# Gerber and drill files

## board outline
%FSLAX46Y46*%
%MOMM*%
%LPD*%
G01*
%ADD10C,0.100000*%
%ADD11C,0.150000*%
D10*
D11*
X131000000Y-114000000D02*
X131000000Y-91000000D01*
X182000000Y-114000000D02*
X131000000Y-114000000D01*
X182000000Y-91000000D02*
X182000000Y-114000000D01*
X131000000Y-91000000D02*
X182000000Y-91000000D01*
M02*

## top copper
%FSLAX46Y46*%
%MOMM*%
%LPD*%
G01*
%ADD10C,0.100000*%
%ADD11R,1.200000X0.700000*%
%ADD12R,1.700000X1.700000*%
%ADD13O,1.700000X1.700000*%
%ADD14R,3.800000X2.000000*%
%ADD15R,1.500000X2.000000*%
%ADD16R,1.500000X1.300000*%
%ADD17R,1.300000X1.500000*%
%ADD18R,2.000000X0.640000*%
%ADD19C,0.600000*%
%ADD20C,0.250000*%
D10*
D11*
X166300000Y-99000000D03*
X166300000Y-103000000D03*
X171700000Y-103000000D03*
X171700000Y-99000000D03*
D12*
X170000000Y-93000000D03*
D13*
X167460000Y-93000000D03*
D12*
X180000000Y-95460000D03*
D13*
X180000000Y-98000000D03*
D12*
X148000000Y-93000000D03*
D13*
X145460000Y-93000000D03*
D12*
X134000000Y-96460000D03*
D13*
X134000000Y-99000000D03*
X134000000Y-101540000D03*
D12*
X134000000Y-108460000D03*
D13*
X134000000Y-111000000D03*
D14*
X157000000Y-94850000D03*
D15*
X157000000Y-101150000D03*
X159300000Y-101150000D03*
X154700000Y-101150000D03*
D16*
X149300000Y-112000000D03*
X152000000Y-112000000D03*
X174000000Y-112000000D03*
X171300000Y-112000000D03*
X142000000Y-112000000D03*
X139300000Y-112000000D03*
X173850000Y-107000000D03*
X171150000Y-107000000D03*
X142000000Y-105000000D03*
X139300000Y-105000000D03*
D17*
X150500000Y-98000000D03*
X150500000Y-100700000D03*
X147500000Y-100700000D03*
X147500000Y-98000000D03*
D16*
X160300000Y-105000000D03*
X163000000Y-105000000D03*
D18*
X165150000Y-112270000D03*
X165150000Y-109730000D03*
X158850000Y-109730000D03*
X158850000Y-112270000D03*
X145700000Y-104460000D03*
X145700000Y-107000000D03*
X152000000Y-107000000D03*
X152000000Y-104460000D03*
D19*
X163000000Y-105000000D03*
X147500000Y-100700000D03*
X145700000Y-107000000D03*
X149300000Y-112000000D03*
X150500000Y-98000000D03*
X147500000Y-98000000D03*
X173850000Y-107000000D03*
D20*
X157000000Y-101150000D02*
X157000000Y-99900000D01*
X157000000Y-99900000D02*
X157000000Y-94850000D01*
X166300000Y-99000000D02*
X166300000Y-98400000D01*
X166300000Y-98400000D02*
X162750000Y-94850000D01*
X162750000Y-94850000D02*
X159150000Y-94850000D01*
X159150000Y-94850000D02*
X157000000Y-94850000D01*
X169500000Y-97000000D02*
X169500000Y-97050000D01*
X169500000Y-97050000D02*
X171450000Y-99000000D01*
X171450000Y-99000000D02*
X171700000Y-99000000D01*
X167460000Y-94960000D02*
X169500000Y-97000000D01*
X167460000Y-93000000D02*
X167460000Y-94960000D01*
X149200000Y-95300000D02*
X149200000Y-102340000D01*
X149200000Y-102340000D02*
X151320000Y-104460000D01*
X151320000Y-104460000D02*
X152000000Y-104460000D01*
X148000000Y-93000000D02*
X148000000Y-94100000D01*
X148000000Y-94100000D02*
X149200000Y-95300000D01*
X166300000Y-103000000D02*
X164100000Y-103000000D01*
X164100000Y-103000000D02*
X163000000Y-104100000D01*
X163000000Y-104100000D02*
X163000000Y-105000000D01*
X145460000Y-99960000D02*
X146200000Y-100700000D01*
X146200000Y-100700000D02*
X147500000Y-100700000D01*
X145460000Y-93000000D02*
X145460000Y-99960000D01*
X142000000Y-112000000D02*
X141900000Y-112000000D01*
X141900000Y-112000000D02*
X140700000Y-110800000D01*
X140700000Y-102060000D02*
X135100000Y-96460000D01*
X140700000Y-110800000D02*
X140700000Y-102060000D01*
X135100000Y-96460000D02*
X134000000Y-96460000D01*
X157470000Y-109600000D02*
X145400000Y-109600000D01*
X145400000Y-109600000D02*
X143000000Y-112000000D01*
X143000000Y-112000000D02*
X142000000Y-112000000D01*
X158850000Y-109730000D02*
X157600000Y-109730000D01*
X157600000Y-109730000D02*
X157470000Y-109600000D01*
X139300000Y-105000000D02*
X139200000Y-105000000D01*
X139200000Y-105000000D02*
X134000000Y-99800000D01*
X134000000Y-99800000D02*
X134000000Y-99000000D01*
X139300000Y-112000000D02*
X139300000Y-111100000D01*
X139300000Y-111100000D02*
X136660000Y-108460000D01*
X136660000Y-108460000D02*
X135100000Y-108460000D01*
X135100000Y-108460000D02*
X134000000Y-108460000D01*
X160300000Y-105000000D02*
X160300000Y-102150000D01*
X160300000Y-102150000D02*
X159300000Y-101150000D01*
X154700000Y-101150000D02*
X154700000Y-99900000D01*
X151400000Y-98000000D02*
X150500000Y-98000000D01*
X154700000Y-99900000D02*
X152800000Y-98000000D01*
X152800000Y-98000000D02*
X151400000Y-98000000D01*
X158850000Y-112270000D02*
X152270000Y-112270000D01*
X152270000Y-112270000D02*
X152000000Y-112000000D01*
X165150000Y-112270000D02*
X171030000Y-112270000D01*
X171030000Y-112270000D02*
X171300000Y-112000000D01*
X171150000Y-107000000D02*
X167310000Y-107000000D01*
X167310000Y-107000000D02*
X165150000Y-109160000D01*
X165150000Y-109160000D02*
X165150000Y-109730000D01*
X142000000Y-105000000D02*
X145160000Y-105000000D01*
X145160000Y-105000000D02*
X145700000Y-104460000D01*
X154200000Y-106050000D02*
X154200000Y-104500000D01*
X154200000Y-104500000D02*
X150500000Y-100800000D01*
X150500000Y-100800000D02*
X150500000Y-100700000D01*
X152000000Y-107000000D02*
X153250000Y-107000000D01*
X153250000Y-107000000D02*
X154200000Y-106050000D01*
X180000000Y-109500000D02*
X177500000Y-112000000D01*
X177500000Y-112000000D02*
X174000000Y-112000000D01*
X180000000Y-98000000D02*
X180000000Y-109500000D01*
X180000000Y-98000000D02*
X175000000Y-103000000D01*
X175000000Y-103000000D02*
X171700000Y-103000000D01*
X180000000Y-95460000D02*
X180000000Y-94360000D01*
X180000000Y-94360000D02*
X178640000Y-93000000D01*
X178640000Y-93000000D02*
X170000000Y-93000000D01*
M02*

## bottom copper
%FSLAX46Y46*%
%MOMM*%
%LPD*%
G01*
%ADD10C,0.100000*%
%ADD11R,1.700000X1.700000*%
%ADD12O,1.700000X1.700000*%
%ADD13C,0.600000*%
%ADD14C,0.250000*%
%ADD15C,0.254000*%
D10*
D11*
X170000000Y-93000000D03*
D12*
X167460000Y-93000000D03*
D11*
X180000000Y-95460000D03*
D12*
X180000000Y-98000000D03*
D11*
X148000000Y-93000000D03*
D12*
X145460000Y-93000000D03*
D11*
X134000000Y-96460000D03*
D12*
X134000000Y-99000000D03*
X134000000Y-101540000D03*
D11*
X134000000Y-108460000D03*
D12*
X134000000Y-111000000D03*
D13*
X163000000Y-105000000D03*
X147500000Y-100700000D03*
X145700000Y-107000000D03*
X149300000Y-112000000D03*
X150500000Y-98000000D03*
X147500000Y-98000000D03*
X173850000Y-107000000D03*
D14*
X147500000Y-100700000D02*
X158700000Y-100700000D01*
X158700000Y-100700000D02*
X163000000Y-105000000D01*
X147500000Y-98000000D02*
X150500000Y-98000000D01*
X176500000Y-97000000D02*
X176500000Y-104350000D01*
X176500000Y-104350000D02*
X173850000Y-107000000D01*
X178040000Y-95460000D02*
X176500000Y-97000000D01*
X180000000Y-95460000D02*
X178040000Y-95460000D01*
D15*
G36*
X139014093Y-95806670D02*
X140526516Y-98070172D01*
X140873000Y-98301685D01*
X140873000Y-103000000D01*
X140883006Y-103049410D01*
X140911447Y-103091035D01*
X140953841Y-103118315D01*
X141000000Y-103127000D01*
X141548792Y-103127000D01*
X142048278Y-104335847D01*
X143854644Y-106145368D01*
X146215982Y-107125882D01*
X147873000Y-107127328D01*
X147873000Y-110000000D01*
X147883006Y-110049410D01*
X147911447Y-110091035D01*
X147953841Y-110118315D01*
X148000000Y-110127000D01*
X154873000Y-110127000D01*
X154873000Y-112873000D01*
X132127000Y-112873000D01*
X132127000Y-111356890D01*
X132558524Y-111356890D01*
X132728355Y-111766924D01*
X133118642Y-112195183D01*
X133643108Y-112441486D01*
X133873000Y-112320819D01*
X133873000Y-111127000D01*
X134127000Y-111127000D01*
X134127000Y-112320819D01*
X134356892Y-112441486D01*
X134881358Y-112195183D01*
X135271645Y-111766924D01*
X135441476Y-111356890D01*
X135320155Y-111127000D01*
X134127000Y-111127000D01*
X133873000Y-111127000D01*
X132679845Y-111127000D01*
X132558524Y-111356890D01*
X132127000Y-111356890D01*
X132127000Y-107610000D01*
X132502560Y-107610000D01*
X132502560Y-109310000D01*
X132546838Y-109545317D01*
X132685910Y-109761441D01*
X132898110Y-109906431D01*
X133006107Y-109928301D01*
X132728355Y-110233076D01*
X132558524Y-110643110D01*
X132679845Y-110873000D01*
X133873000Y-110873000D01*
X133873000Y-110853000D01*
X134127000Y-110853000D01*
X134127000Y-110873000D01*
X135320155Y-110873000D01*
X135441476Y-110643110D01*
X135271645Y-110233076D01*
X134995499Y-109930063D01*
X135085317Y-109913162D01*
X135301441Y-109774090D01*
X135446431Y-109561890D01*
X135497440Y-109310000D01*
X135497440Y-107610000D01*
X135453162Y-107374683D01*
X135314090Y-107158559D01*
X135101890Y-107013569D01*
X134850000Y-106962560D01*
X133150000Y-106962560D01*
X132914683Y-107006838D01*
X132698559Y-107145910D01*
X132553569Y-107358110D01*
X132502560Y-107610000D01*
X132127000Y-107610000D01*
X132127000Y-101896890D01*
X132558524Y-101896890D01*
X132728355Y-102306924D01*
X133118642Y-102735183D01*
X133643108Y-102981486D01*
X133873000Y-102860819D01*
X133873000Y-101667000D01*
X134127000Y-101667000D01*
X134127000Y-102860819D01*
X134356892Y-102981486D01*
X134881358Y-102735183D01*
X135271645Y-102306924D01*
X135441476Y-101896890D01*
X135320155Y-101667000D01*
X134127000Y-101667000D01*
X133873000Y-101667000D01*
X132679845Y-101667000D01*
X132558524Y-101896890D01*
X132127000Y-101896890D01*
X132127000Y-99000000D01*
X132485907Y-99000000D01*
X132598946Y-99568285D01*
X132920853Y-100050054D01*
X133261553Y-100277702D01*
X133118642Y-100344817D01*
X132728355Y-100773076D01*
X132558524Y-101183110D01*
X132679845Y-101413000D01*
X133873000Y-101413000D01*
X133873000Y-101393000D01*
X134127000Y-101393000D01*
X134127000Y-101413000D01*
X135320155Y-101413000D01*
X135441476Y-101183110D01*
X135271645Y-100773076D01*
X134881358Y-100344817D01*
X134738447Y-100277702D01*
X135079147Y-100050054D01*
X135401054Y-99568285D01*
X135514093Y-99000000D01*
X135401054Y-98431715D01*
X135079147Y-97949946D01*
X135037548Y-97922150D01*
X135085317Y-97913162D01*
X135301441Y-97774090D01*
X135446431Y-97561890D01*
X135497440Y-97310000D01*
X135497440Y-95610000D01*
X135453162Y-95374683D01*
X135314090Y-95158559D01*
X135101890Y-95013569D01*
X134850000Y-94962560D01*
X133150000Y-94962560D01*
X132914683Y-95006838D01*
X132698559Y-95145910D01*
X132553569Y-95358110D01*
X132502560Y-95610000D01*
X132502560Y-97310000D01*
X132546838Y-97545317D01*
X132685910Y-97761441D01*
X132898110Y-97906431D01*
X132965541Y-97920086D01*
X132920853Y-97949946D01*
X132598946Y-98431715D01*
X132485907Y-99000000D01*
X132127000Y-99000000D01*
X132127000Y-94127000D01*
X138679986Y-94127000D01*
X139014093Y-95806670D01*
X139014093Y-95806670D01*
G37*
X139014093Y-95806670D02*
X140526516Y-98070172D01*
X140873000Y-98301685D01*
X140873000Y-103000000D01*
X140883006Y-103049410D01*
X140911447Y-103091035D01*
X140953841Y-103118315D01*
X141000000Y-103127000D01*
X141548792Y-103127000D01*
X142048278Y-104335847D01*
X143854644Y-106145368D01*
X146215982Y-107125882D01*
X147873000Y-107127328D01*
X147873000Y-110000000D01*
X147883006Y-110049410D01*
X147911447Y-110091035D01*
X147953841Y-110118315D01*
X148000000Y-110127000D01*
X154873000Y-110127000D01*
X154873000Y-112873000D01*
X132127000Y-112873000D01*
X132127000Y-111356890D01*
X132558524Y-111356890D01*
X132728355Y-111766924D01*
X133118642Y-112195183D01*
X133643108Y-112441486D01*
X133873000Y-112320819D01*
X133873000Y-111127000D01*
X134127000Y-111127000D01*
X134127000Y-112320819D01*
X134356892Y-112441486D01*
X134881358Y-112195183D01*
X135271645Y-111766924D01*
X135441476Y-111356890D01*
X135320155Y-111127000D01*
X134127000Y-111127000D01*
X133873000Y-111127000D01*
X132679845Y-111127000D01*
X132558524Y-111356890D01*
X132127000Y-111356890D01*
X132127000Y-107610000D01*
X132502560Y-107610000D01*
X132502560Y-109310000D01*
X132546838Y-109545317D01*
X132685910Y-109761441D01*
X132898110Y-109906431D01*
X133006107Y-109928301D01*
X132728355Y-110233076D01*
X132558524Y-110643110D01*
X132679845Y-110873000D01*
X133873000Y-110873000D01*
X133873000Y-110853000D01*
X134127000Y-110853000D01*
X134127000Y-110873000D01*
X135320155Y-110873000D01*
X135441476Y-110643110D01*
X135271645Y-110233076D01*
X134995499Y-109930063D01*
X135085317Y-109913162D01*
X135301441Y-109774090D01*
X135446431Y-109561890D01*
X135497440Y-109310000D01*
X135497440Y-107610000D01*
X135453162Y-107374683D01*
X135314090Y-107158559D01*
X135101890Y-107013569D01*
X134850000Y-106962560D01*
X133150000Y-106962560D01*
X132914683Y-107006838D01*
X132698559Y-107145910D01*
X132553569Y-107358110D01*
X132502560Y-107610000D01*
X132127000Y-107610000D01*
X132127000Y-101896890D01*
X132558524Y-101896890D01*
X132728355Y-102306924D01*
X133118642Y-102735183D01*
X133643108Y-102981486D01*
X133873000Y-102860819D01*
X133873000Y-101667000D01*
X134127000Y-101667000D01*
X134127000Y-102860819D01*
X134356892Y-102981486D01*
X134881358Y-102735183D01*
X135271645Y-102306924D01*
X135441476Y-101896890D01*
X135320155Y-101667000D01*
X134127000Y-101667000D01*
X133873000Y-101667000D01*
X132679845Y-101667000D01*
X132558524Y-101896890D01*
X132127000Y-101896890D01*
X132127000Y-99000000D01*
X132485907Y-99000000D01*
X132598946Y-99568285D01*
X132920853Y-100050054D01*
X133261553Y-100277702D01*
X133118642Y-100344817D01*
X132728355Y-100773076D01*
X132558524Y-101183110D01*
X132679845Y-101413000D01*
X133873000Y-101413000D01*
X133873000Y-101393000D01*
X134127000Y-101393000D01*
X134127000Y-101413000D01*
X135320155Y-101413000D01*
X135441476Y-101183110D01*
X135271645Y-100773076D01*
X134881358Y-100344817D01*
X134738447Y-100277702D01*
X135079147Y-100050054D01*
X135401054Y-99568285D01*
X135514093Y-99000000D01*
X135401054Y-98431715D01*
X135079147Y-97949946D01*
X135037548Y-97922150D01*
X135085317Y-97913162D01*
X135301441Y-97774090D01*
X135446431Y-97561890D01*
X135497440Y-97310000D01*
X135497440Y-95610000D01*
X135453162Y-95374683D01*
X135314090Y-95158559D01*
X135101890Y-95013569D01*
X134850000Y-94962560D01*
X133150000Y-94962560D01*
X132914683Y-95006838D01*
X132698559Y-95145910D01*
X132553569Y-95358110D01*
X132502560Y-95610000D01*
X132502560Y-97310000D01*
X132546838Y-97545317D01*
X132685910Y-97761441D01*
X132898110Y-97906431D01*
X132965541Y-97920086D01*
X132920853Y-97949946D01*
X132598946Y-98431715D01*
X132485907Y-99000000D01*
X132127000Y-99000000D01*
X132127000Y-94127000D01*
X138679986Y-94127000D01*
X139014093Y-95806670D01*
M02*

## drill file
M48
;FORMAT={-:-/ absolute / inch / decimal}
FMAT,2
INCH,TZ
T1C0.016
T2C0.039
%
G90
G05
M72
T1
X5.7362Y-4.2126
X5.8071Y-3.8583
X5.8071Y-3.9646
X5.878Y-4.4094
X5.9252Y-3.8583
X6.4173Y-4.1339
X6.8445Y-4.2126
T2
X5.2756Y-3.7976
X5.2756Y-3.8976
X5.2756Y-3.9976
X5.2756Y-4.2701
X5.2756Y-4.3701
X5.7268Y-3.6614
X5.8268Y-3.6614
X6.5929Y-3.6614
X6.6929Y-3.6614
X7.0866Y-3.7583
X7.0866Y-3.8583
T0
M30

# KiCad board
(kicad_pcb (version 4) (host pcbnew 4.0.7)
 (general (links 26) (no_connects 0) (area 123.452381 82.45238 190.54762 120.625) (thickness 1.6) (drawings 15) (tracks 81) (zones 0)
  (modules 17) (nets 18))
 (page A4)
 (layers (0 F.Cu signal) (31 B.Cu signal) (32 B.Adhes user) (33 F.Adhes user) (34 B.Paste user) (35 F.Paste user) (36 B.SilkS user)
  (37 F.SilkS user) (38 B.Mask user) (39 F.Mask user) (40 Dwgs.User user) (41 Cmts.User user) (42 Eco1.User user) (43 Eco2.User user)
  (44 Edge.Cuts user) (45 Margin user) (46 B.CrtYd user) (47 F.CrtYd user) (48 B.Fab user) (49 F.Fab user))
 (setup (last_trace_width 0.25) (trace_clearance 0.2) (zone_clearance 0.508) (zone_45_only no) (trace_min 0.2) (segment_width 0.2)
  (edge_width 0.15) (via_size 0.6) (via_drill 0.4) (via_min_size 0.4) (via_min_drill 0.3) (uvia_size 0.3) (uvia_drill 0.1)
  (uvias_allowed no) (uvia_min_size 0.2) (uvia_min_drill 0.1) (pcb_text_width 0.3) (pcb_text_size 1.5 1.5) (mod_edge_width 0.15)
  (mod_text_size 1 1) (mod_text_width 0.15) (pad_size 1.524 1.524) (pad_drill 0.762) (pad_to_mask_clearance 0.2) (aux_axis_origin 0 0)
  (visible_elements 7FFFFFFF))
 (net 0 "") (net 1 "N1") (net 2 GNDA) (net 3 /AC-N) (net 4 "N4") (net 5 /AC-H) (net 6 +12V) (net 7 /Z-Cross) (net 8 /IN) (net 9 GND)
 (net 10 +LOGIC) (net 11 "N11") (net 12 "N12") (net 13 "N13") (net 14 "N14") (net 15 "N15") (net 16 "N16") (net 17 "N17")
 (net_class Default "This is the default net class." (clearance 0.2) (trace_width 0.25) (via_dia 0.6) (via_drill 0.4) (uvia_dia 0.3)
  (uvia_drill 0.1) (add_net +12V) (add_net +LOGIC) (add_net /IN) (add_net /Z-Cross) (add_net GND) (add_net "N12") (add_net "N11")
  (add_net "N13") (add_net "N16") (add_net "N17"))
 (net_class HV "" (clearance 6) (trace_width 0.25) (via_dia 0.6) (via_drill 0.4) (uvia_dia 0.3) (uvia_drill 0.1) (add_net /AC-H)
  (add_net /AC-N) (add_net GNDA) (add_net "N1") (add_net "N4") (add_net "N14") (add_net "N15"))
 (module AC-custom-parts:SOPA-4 (layer F.Cu) (at 169 101)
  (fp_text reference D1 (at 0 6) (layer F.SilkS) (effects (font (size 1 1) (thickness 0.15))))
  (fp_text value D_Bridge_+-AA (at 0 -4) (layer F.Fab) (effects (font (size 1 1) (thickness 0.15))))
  (pad 1 smd rect (at -2.7 -2) (size 1.2 0.7) (layers F.Cu F.Paste F.Mask) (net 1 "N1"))
  (pad 2 smd rect (at -2.7 2) (size 1.2 0.7) (layers F.Cu F.Paste F.Mask) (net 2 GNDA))
  (pad 3 smd rect (at 2.7 2) (size 1.2 0.7) (layers F.Cu F.Paste F.Mask) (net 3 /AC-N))
  (pad 4 smd rect (at 2.7 -2) (size 1.2 0.7) (layers F.Cu F.Paste F.Mask) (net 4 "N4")))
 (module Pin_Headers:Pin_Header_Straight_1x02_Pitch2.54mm (layer F.Cu) (at 170 93 270)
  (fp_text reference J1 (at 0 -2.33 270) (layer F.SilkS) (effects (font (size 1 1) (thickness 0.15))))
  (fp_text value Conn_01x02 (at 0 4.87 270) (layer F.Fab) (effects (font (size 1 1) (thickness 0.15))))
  (pad 1 thru_hole rect (at 0 0 270) (size 1.7 1.7) (drill 1) (layers *.Cu *.Mask) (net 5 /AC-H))
  (pad 2 thru_hole oval (at 0 2.54 270) (size 1.7 1.7) (drill 1) (layers *.Cu *.Mask) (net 4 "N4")))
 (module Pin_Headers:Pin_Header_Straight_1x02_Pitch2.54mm (layer F.Cu) (at 180 95.46)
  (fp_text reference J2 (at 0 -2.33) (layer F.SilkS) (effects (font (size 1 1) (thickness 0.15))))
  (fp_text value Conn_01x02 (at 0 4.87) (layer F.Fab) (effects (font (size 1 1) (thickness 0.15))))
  (pad 1 thru_hole rect (at 0 0) (size 1.7 1.7) (drill 1) (layers *.Cu *.Mask) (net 5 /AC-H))
  (pad 2 thru_hole oval (at 0 2.54) (size 1.7 1.7) (drill 1) (layers *.Cu *.Mask) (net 3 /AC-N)))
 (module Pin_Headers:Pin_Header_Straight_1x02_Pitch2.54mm (layer F.Cu) (at 148 93 270)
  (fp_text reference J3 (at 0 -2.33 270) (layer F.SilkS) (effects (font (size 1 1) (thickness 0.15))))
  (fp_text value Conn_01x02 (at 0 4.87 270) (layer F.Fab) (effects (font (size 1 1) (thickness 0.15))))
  (pad 1 thru_hole rect (at 0 0 270) (size 1.7 1.7) (drill 1) (layers *.Cu *.Mask) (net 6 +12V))
  (pad 2 thru_hole oval (at 0 2.54 270) (size 1.7 1.7) (drill 1) (layers *.Cu *.Mask) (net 2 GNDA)))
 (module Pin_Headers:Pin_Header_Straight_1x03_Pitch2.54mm (layer F.Cu) (at 134 96.46)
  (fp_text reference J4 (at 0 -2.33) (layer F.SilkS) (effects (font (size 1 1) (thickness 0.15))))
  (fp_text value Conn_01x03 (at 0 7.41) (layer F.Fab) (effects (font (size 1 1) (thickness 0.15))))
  (pad 1 thru_hole rect (at 0 0) (size 1.7 1.7) (drill 1) (layers *.Cu *.Mask) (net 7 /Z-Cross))
  (pad 2 thru_hole oval (at 0 2.54) (size 1.7 1.7) (drill 1) (layers *.Cu *.Mask) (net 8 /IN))
  (pad 3 thru_hole oval (at 0 5.08) (size 1.7 1.7) (drill 1) (layers *.Cu *.Mask) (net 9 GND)))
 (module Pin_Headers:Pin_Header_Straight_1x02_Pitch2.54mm (layer F.Cu) (at 134 108.46)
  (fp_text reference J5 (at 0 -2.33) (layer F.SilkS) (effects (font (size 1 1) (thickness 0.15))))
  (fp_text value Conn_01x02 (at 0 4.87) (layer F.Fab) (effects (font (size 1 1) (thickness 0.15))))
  (pad 1 thru_hole rect (at 0 0) (size 1.7 1.7) (drill 1) (layers *.Cu *.Mask) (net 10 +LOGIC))
  (pad 2 thru_hole oval (at 0 2.54) (size 1.7 1.7) (drill 1) (layers *.Cu *.Mask) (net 9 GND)))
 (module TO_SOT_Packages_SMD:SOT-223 (layer F.Cu) (at 157 98 90)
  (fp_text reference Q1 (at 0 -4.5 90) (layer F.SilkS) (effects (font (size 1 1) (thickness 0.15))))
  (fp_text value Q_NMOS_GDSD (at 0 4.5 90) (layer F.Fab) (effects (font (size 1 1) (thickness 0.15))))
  (pad 4 smd rect (at 3.15 0 90) (size 2 3.8) (layers F.Cu F.Paste F.Mask) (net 1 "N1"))
  (pad 2 smd rect (at -3.15 0 90) (size 2 1.5) (layers F.Cu F.Paste F.Mask) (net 1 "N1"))
  (pad 3 smd rect (at -3.15 2.3 90) (size 2 1.5) (layers F.Cu F.Paste F.Mask) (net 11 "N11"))
  (pad 1 smd rect (at -3.15 -2.3 90) (size 2 1.5) (layers F.Cu F.Paste F.Mask) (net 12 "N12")))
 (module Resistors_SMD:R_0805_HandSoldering (layer F.Cu) (at 150.65 112)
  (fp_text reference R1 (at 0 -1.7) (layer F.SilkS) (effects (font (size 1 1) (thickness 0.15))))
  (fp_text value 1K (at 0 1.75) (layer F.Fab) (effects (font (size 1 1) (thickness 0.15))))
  (pad 1 smd rect (at -1.35 0) (size 1.5 1.3) (layers F.Cu F.Paste F.Mask) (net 9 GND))
  (pad 2 smd rect (at 1.35 0) (size 1.5 1.3) (layers F.Cu F.Paste F.Mask) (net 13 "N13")))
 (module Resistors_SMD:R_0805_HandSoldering (layer F.Cu) (at 172.65 112 180)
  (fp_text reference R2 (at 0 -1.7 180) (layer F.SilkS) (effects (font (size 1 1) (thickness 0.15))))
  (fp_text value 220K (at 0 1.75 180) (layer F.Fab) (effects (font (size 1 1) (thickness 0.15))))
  (pad 1 smd rect (at -1.35 0 180) (size 1.5 1.3) (layers F.Cu F.Paste F.Mask) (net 3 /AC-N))
  (pad 2 smd rect (at 1.35 0 180) (size 1.5 1.3) (layers F.Cu F.Paste F.Mask) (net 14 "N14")))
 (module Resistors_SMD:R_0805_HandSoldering (layer F.Cu) (at 140.65 112 180)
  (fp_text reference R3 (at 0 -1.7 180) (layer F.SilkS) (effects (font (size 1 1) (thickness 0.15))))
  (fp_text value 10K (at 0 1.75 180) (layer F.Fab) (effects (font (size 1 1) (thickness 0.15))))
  (pad 1 smd rect (at -1.35 0 180) (size 1.5 1.3) (layers F.Cu F.Paste F.Mask) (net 7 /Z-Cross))
  (pad 2 smd rect (at 1.35 0 180) (size 1.5 1.3) (layers F.Cu F.Paste F.Mask) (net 10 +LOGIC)))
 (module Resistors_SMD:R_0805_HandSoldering (layer F.Cu) (at 172.5 107 180)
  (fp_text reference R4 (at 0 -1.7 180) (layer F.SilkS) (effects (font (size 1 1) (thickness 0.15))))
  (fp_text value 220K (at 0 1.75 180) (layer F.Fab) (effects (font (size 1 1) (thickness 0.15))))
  (pad 1 smd rect (at -1.35 0 180) (size 1.5 1.3) (layers F.Cu F.Paste F.Mask) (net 5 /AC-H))
  (pad 2 smd rect (at 1.35 0 180) (size 1.5 1.3) (layers F.Cu F.Paste F.Mask) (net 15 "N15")))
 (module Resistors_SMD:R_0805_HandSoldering (layer F.Cu) (at 140.65 105 180)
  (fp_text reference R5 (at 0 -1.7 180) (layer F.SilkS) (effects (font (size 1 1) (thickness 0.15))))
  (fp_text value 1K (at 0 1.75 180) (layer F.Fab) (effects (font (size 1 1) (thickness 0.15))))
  (pad 1 smd rect (at -1.35 0 180) (size 1.5 1.3) (layers F.Cu F.Paste F.Mask) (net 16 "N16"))
  (pad 2 smd rect (at 1.35 0 180) (size 1.5 1.3) (layers F.Cu F.Paste F.Mask) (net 8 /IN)))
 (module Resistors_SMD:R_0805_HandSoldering (layer F.Cu) (at 150.5 99.35 270)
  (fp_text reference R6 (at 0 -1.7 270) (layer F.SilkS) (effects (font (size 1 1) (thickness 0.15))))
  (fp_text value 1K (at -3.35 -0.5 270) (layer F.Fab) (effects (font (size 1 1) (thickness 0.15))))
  (pad 1 smd rect (at -1.35 0 270) (size 1.5 1.3) (layers F.Cu F.Paste F.Mask) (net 12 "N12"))
  (pad 2 smd rect (at 1.35 0 270) (size 1.5 1.3) (layers F.Cu F.Paste F.Mask) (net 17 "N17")))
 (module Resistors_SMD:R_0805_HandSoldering (layer F.Cu) (at 147.5 99.35 90)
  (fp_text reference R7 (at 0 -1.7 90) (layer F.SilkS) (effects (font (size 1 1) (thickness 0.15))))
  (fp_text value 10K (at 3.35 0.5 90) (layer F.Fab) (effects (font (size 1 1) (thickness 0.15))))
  (pad 1 smd rect (at -1.35 0 90) (size 1.5 1.3) (layers F.Cu F.Paste F.Mask) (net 2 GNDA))
  (pad 2 smd rect (at 1.35 0 90) (size 1.5 1.3) (layers F.Cu F.Paste F.Mask) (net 12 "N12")))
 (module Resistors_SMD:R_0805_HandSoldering (layer F.Cu) (at 161.65 105)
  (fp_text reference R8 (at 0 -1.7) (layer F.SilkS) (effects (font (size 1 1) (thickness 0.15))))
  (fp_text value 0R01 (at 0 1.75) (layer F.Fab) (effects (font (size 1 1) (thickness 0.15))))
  (pad 1 smd rect (at -1.35 0) (size 1.5 1.3) (layers F.Cu F.Paste F.Mask) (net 11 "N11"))
  (pad 2 smd rect (at 1.35 0) (size 1.5 1.3) (layers F.Cu F.Paste F.Mask) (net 2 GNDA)))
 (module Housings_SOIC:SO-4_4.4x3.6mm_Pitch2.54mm (layer F.Cu) (at 162 111 180)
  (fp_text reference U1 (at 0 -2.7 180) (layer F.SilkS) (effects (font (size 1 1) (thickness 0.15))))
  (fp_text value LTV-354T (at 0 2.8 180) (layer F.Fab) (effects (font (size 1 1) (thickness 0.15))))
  (pad 1 smd rect (at -3.15 -1.27 180) (size 2 0.64) (layers F.Cu F.Paste F.Mask) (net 14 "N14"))
  (pad 2 smd rect (at -3.15 1.27 180) (size 2 0.64) (layers F.Cu F.Paste F.Mask) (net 15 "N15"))
  (pad 3 smd rect (at 3.15 1.27 180) (size 2 0.64) (layers F.Cu F.Paste F.Mask) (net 7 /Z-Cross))
  (pad 4 smd rect (at 3.15 -1.27 180) (size 2 0.64) (layers F.Cu F.Paste F.Mask) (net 13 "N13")))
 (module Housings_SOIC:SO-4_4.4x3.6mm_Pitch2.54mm (layer F.Cu) (at 148.85 105.73)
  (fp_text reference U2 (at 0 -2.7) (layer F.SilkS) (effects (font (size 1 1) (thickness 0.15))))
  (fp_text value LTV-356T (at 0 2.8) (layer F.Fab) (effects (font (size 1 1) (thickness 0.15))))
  (pad 1 smd rect (at -3.15 -1.27) (size 2 0.64) (layers F.Cu F.Paste F.Mask) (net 16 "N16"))
  (pad 2 smd rect (at -3.15 1.27) (size 2 0.64) (layers F.Cu F.Paste F.Mask) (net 9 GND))
  (pad 3 smd rect (at 3.15 1.27) (size 2 0.64) (layers F.Cu F.Paste F.Mask) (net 17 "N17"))
  (pad 4 smd rect (at 3.15 -1.27) (size 2 0.64) (layers F.Cu F.Paste F.Mask) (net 6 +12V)))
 (gr_line (start 131 114) (end 131 91) (layer Edge.Cuts) (width 0.15))
 (gr_line (start 182 114) (end 131 114) (layer Edge.Cuts) (width 0.15))
 (gr_line (start 182 91) (end 182 114) (layer Edge.Cuts) (width 0.15))
 (gr_line (start 131 91) (end 182 91) (layer Edge.Cuts) (width 0.15))
 (segment (start 157 101.15) (end 157 99.9) (width 0.25) (layer F.Cu) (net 1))
 (segment (start 157 99.9) (end 157 94.85) (width 0.25) (layer F.Cu) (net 1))
 (segment (start 166.3 99) (end 166.3 98.4) (width 0.25) (layer F.Cu) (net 1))
 (segment (start 166.3 98.4) (end 162.75 94.85) (width 0.25) (layer F.Cu) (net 1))
 (segment (start 162.75 94.85) (end 159.15 94.85) (width 0.25) (layer F.Cu) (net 1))
 (segment (start 159.15 94.85) (end 157 94.85) (width 0.25) (layer F.Cu) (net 1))
 (segment (start 169.5 97) (end 169.5 97.05) (width 0.25) (layer F.Cu) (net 4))
 (segment (start 169.5 97.05) (end 171.45 99) (width 0.25) (layer F.Cu) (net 4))
 (segment (start 171.45 99) (end 171.7 99) (width 0.25) (layer F.Cu) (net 4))
 (segment (start 167.46 94.96) (end 169.5 97) (width 0.25) (layer F.Cu) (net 4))
 (segment (start 167.46 93) (end 167.46 94.96) (width 0.25) (layer F.Cu) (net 4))
 (segment (start 149.2 95.3) (end 149.2 102.34) (width 0.25) (layer F.Cu) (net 6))
 (segment (start 149.2 102.34) (end 151.32 104.46) (width 0.25) (layer F.Cu) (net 6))
 (segment (start 151.32 104.46) (end 152 104.46) (width 0.25) (layer F.Cu) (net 6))
 (segment (start 148 93) (end 148 94.1) (width 0.25) (layer F.Cu) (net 6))
 (segment (start 148 94.1) (end 149.2 95.3) (width 0.25) (layer F.Cu) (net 6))
 (segment (start 147.5 100.7) (end 158.7 100.7) (width 0.25) (layer B.Cu) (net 2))
 (via (at 163 105) (size 0.6) (drill 0.4) (layers F.Cu B.Cu) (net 2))
 (segment (start 158.7 100.7) (end 163 105) (width 0.25) (layer B.Cu) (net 2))
 (via (at 147.5 100.7) (size 0.6) (drill 0.4) (layers F.Cu B.Cu) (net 2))
 (segment (start 166.3 103) (end 164.1 103) (width 0.25) (layer F.Cu) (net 2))
 (segment (start 164.1 103) (end 163 104.1) (width 0.25) (layer F.Cu) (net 2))
 (segment (start 163 104.1) (end 163 105) (width 0.25) (layer F.Cu) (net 2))
 (segment (start 145.46 99.96) (end 146.2 100.7) (width 0.25) (layer F.Cu) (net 2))
 (segment (start 146.2 100.7) (end 147.5 100.7) (width 0.25) (layer F.Cu) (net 2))
 (segment (start 145.46 93) (end 145.46 99.96) (width 0.25) (layer F.Cu) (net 2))
 (segment (start 142 112) (end 141.9 112) (width 0.25) (layer F.Cu) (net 7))
 (segment (start 141.9 112) (end 140.7 110.8) (width 0.25) (layer F.Cu) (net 7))
 (segment (start 140.7 102.06) (end 135.1 96.46) (width 0.25) (layer F.Cu) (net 7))
 (segment (start 140.7 110.8) (end 140.7 102.06) (width 0.25) (layer F.Cu) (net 7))
 (segment (start 135.1 96.46) (end 134 96.46) (width 0.25) (layer F.Cu) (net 7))
 (segment (start 157.47 109.6) (end 145.4 109.6) (width 0.25) (layer F.Cu) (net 7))
 (segment (start 145.4 109.6) (end 143 112) (width 0.25) (layer F.Cu) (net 7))
 (segment (start 143 112) (end 142 112) (width 0.25) (layer F.Cu) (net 7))
 (segment (start 158.85 109.73) (end 157.6 109.73) (width 0.25) (layer F.Cu) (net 7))
 (segment (start 157.6 109.73) (end 157.47 109.6) (width 0.25) (layer F.Cu) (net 7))
 (segment (start 139.3 105) (end 139.2 105) (width 0.25) (layer F.Cu) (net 8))
 (segment (start 139.2 105) (end 134 99.8) (width 0.25) (layer F.Cu) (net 8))
 (segment (start 134 99.8) (end 134 99) (width 0.25) (layer F.Cu) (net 8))
 (via (at 145.7 107) (size 0.6) (drill 0.4) (layers F.Cu B.Cu) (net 9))
 (via (at 149.3 112) (size 0.6) (drill 0.4) (layers F.Cu B.Cu) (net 9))
 (segment (start 139.3 112) (end 139.3 111.1) (width 0.25) (layer F.Cu) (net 10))
 (segment (start 139.3 111.1) (end 136.66 108.46) (width 0.25) (layer F.Cu) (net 10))
 (segment (start 136.66 108.46) (end 135.1 108.46) (width 0.25) (layer F.Cu) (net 10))
 (segment (start 135.1 108.46) (end 134 108.46) (width 0.25) (layer F.Cu) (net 10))
 (segment (start 160.3 105) (end 160.3 102.15) (width 0.25) (layer F.Cu) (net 11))
 (segment (start 160.3 102.15) (end 159.3 101.15) (width 0.25) (layer F.Cu) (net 11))
 (segment (start 147.5 98) (end 150.5 98) (width 0.25) (layer B.Cu) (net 12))
 (via (at 150.5 98) (size 0.6) (drill 0.4) (layers F.Cu B.Cu) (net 12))
 (via (at 147.5 98) (size 0.6) (drill 0.4) (layers F.Cu B.Cu) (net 12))
 (segment (start 154.7 101.15) (end 154.7 99.9) (width 0.25) (layer F.Cu) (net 12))
 (segment (start 151.4 98) (end 150.5 98) (width 0.25) (layer F.Cu) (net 12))
 (segment (start 154.7 99.9) (end 152.8 98) (width 0.25) (layer F.Cu) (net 12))
 (segment (start 152.8 98) (end 151.4 98) (width 0.25) (layer F.Cu) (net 12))
 (segment (start 158.85 112.27) (end 152.27 112.27) (width 0.25) (layer F.Cu) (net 13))
 (segment (start 152.27 112.27) (end 152 112) (width 0.25) (layer F.Cu) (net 13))
 (segment (start 165.15 112.27) (end 171.03 112.27) (width 0.25) (layer F.Cu) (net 14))
 (segment (start 171.03 112.27) (end 171.3 112) (width 0.25) (layer F.Cu) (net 14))
 (segment (start 171.15 107) (end 167.31 107) (width 0.25) (layer F.Cu) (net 15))
 (segment (start 167.31 107) (end 165.15 109.16) (width 0.25) (layer F.Cu) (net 15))
 (segment (start 165.15 109.16) (end 165.15 109.73) (width 0.25) (layer F.Cu) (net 15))
 (segment (start 142 105) (end 145.16 105) (width 0.25) (layer F.Cu) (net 16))
 (segment (start 145.16 105) (end 145.7 104.46) (width 0.25) (layer F.Cu) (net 16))
 (segment (start 154.2 106.05) (end 154.2 104.5) (width 0.25) (layer F.Cu) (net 17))
 (segment (start 154.2 104.5) (end 150.5 100.8) (width 0.25) (layer F.Cu) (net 17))
 (segment (start 150.5 100.8) (end 150.5 100.7) (width 0.25) (layer F.Cu) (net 17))
 (segment (start 152 107) (end 153.25 107) (width 0.25) (layer F.Cu) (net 17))
 (segment (start 153.25 107) (end 154.2 106.05) (width 0.25) (layer F.Cu) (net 17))
 (segment (start 180 109.5) (end 177.5 112) (width 0.25) (layer F.Cu) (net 3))
 (segment (start 177.5 112) (end 174 112) (width 0.25) (layer F.Cu) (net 3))
 (segment (start 180 98) (end 180 109.5) (width 0.25) (layer F.Cu) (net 3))
 (segment (start 180 98) (end 175 103) (width 0.25) (layer F.Cu) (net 3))
 (segment (start 175 103) (end 171.7 103) (width 0.25) (layer F.Cu) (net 3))
 (segment (start 176.5 97) (end 176.5 104.35) (width 0.25) (layer B.Cu) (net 5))
 (segment (start 176.5 104.35) (end 173.85 107) (width 0.25) (layer B.Cu) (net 5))
 (via (at 173.85 107) (size 0.6) (drill 0.4) (layers F.Cu B.Cu) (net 5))
 (segment (start 178.04 95.46) (end 176.5 97) (width 0.25) (layer B.Cu) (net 5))
 (segment (start 180 95.46) (end 178.04 95.46) (width 0.25) (layer B.Cu) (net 5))
 (segment (start 180 95.46) (end 180 94.36) (width 0.25) (layer F.Cu) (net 5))
 (segment (start 180 94.36) (end 178.64 93) (width 0.25) (layer F.Cu) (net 5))
 (segment (start 178.64 93) (end 170 93) (width 0.25) (layer F.Cu) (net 5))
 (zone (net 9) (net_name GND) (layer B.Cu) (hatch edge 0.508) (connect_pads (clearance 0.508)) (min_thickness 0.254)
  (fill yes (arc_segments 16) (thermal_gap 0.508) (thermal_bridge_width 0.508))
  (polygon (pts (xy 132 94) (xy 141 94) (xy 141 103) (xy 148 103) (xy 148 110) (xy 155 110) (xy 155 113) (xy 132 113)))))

